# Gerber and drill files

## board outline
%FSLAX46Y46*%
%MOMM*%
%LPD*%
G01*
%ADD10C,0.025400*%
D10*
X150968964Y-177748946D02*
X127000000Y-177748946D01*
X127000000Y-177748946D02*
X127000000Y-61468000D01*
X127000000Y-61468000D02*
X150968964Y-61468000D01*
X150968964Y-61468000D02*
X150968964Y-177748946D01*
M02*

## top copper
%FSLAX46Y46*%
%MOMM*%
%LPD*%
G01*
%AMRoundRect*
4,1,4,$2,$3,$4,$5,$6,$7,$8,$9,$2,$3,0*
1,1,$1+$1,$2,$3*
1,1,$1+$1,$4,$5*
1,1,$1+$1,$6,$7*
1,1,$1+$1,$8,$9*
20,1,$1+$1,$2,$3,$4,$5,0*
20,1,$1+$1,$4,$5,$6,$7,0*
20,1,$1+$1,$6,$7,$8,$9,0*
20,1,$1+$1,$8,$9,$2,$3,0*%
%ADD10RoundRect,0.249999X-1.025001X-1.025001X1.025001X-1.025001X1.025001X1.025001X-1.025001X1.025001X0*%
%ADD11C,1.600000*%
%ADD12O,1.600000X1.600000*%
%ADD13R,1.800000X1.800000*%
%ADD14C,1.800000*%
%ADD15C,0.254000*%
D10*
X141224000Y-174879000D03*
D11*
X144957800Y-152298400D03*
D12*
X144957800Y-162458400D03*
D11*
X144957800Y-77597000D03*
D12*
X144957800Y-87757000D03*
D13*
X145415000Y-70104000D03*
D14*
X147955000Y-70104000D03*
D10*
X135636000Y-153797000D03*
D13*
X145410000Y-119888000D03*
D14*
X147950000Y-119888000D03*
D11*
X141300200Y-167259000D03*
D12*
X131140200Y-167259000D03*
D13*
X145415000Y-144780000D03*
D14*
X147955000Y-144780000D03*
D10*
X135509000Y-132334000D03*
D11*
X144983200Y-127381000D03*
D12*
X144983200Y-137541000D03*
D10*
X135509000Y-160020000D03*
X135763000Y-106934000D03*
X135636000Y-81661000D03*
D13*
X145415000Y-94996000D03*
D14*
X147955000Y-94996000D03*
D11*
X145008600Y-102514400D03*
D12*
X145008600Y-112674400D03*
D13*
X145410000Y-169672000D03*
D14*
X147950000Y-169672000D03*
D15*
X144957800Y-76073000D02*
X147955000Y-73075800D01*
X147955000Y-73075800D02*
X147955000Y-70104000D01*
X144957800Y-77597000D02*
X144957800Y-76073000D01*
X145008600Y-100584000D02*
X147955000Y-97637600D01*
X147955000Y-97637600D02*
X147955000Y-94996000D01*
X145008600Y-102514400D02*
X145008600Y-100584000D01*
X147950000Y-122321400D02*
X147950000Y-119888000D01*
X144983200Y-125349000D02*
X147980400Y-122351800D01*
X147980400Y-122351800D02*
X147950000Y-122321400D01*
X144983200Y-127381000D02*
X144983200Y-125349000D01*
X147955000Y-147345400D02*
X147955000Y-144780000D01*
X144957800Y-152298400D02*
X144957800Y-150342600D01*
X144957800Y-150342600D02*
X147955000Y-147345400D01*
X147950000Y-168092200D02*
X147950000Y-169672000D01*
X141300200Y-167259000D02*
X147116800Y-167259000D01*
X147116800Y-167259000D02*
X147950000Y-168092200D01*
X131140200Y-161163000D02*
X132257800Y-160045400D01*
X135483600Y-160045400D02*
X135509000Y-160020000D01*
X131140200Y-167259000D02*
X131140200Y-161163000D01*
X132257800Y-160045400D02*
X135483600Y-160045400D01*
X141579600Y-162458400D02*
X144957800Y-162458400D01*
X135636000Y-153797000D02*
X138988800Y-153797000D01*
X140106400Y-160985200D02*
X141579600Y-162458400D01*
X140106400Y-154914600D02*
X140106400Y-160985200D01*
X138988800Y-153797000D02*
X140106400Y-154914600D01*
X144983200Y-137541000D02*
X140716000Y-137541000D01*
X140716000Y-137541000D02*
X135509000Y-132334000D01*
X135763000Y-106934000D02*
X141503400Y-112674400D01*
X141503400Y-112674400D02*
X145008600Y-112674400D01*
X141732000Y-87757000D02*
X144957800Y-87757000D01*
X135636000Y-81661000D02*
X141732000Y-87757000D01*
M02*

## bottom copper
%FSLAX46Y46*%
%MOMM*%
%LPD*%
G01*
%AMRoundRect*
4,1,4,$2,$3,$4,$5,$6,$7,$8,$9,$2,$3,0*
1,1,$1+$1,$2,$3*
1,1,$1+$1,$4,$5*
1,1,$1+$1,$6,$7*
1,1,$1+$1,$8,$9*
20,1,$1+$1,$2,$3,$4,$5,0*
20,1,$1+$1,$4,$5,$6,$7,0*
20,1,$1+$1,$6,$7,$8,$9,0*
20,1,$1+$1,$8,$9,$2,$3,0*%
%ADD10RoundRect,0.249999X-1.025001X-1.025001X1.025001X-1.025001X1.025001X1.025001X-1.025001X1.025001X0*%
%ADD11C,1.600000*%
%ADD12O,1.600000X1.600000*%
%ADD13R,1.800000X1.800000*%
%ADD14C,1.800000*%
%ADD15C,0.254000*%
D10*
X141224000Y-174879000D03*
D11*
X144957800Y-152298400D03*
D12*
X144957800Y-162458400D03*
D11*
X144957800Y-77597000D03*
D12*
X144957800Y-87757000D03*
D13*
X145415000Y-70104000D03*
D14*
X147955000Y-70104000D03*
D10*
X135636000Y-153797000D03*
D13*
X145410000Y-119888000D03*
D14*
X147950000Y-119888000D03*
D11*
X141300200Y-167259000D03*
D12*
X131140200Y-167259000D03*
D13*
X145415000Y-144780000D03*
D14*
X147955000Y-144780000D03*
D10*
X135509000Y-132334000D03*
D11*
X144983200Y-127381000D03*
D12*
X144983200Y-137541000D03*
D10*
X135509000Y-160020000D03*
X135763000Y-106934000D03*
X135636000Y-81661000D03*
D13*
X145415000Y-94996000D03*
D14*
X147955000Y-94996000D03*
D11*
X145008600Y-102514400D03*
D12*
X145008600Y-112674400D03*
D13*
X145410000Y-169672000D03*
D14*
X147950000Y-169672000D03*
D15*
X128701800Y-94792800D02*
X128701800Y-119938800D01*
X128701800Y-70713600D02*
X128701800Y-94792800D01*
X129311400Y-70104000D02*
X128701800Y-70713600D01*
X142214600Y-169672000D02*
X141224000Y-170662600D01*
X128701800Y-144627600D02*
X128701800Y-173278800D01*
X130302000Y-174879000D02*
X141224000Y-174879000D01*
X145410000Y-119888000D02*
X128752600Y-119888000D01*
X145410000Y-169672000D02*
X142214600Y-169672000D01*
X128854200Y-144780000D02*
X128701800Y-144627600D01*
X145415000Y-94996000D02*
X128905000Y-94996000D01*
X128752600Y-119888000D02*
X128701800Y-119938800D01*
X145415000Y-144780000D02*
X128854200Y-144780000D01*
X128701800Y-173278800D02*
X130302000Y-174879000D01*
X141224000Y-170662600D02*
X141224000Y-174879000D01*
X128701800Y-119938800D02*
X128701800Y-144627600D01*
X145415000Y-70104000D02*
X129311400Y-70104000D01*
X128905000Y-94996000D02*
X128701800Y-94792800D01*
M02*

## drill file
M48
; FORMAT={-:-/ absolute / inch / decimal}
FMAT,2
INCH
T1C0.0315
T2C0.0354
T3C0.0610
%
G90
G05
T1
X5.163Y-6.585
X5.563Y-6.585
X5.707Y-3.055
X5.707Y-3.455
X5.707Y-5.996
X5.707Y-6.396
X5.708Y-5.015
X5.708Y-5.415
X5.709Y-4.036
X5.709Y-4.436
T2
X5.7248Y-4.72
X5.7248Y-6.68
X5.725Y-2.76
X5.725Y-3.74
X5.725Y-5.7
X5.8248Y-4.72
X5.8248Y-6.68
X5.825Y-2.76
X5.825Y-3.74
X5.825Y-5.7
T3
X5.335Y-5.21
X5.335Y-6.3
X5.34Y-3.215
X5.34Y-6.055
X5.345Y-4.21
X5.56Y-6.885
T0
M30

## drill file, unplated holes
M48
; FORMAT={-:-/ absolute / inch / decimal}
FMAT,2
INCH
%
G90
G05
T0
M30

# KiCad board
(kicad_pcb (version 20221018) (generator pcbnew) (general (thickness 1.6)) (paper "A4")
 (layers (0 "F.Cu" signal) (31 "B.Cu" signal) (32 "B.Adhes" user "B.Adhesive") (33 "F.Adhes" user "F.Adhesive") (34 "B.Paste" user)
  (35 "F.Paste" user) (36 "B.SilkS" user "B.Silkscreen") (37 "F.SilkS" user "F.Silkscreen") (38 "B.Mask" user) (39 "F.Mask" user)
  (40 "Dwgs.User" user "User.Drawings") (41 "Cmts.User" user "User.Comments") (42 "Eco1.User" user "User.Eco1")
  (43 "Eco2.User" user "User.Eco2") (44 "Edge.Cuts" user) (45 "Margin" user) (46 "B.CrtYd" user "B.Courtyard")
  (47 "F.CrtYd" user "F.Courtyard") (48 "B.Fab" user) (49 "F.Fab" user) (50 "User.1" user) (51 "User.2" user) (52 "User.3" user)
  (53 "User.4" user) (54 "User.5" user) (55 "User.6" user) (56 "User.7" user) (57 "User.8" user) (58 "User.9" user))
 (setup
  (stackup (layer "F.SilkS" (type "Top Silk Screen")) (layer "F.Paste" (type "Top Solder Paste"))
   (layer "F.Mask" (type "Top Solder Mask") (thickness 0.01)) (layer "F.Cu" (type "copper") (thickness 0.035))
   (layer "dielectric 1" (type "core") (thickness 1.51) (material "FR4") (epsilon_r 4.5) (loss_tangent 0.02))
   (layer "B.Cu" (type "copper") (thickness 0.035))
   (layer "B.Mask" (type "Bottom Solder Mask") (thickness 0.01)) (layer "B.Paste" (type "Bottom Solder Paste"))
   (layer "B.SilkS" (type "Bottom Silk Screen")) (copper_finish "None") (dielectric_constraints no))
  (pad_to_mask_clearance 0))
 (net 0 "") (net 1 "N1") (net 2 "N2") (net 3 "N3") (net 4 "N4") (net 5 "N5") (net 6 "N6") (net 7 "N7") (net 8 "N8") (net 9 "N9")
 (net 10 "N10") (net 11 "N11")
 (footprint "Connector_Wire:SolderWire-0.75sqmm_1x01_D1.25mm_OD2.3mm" (layer "F.Cu") (at 141.224 174.879)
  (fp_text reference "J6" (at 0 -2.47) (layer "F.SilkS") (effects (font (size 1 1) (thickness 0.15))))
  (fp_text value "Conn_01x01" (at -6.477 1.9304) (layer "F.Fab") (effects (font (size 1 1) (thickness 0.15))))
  (pad "1" thru_hole roundrect (at 0 0) (size 2.55 2.55) (drill 1.55) (layers "*.Cu" "*.Mask") (roundrect_rratio 0.09803882353) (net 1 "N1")))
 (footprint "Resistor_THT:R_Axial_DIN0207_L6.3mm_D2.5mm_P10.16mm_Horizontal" (layer "F.Cu") (at 144.9578 152.2984 -90)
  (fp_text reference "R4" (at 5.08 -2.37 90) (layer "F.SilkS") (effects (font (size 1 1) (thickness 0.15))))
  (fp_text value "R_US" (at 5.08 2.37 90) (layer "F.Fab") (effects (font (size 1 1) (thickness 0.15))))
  (pad "1" thru_hole circle (at 0 0 270) (size 1.6 1.6) (drill 0.8) (layers "*.Cu" "*.Mask") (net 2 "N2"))
  (pad "2" thru_hole oval (at 10.16 0 270) (size 1.6 1.6) (drill 0.8) (layers "*.Cu" "*.Mask") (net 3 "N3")))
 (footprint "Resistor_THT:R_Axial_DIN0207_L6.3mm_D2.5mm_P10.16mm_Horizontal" (layer "F.Cu") (at 144.9578 77.597 -90)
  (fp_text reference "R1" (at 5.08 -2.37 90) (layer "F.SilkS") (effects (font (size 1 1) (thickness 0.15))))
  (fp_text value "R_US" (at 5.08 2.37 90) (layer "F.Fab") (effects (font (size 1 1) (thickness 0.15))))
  (pad "1" thru_hole circle (at 0 0 270) (size 1.6 1.6) (drill 0.8) (layers "*.Cu" "*.Mask") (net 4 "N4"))
  (pad "2" thru_hole oval (at 10.16 0 270) (size 1.6 1.6) (drill 0.8) (layers "*.Cu" "*.Mask") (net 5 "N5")))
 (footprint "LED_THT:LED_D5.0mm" (layer "F.Cu") (at 145.415 70.104)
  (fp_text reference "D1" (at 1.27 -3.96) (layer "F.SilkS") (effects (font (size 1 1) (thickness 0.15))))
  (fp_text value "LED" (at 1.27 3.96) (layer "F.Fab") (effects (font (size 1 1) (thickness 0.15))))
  (pad "1" thru_hole rect (at 0 0) (size 1.8 1.8) (drill 0.9) (layers "*.Cu" "*.Mask") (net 1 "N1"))
  (pad "2" thru_hole circle (at 2.54 0) (size 1.8 1.8) (drill 0.9) (layers "*.Cu" "*.Mask") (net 4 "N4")))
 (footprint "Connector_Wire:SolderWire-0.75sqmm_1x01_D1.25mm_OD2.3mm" (layer "F.Cu") (at 135.636 153.797)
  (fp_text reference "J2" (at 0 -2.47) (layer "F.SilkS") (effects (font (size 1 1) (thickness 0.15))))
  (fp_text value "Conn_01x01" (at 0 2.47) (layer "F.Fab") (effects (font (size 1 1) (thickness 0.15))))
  (pad "1" thru_hole roundrect (at 0 0) (size 2.55 2.55) (drill 1.55) (layers "*.Cu" "*.Mask") (roundrect_rratio 0.09803882353) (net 3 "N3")))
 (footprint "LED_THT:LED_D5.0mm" (layer "F.Cu") (at 145.41 119.888)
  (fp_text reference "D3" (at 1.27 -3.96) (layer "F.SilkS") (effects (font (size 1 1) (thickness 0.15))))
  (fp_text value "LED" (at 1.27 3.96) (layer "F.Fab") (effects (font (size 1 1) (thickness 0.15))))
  (pad "1" thru_hole rect (at 0 0) (size 1.8 1.8) (drill 0.9) (layers "*.Cu" "*.Mask") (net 1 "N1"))
  (pad "2" thru_hole circle (at 2.54 0) (size 1.8 1.8) (drill 0.9) (layers "*.Cu" "*.Mask") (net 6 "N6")))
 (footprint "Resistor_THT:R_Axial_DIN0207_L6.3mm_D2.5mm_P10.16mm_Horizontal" (layer "F.Cu") (at 141.3002 167.259 180)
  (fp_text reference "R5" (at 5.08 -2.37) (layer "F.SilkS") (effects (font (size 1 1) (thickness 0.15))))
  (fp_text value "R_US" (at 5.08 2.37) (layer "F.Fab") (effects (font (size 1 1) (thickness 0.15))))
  (pad "1" thru_hole circle (at 0 0 180) (size 1.6 1.6) (drill 0.8) (layers "*.Cu" "*.Mask") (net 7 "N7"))
  (pad "2" thru_hole oval (at 10.16 0 180) (size 1.6 1.6) (drill 0.8) (layers "*.Cu" "*.Mask") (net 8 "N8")))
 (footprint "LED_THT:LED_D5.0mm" (layer "F.Cu") (at 145.415 144.78)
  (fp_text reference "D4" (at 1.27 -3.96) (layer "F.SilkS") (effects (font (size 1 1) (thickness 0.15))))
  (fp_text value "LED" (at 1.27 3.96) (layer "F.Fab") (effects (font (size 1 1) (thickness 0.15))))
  (pad "1" thru_hole rect (at 0 0) (size 1.8 1.8) (drill 0.9) (layers "*.Cu" "*.Mask") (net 1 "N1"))
  (pad "2" thru_hole circle (at 2.54 0) (size 1.8 1.8) (drill 0.9) (layers "*.Cu" "*.Mask") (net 2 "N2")))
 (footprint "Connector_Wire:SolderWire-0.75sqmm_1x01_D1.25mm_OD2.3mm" (layer "F.Cu") (at 135.509 132.334)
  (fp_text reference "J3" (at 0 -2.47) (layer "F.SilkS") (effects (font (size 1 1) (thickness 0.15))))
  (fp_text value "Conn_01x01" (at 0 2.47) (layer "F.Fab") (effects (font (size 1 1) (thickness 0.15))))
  (pad "1" thru_hole roundrect (at 0 0) (size 2.55 2.55) (drill 1.55) (layers "*.Cu" "*.Mask") (roundrect_rratio 0.09803882353) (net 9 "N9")))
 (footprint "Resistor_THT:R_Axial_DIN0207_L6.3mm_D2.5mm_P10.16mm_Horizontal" (layer "F.Cu") (at 144.9832 127.381 -90)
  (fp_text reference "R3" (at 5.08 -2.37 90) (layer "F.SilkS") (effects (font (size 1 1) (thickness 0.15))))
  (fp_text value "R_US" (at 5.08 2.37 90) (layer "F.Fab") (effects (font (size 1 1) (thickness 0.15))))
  (pad "1" thru_hole circle (at 0 0 270) (size 1.6 1.6) (drill 0.8) (layers "*.Cu" "*.Mask") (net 6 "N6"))
  (pad "2" thru_hole oval (at 10.16 0 270) (size 1.6 1.6) (drill 0.8) (layers "*.Cu" "*.Mask") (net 9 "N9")))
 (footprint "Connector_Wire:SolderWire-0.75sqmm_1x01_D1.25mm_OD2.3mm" (layer "F.Cu") (at 135.509 160.02)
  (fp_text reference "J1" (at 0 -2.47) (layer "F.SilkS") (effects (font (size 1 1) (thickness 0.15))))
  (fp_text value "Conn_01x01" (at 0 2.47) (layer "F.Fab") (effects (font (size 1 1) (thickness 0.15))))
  (pad "1" thru_hole roundrect (at 0 0) (size 2.55 2.55) (drill 1.55) (layers "*.Cu" "*.Mask") (roundrect_rratio 0.09803882353) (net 8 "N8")))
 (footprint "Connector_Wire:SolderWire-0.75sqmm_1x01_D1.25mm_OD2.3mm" (layer "F.Cu") (at 135.763 106.934)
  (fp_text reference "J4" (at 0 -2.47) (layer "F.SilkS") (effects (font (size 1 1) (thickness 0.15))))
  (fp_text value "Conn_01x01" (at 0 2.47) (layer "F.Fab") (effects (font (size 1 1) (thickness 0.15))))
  (pad "1" thru_hole roundrect (at 0 0) (size 2.55 2.55) (drill 1.55) (layers "*.Cu" "*.Mask") (roundrect_rratio 0.09803882353)
   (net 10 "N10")))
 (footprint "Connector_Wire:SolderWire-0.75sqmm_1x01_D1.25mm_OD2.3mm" (layer "F.Cu") (at 135.636 81.661)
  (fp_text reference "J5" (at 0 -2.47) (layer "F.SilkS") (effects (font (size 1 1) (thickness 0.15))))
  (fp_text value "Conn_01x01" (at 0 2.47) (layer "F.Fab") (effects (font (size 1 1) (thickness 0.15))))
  (pad "1" thru_hole roundrect (at 0 0) (size 2.55 2.55) (drill 1.55) (layers "*.Cu" "*.Mask") (roundrect_rratio 0.09803882353) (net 5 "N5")))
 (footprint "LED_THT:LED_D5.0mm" (layer "F.Cu") (at 145.415 94.996)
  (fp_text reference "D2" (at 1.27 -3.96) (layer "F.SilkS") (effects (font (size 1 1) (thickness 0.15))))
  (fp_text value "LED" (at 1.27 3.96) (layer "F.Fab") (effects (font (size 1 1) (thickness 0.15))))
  (pad "1" thru_hole rect (at 0 0) (size 1.8 1.8) (drill 0.9) (layers "*.Cu" "*.Mask") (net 1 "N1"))
  (pad "2" thru_hole circle (at 2.54 0) (size 1.8 1.8) (drill 0.9) (layers "*.Cu" "*.Mask") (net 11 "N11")))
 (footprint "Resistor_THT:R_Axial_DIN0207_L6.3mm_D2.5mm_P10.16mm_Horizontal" (layer "F.Cu") (at 145.0086 102.5144 -90)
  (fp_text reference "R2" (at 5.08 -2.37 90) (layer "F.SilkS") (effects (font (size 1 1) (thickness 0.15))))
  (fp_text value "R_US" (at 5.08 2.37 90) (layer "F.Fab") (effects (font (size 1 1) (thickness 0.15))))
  (pad "1" thru_hole circle (at 0 0 270) (size 1.6 1.6) (drill 0.8) (layers "*.Cu" "*.Mask") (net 11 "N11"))
  (pad "2" thru_hole oval (at 10.16 0 270) (size 1.6 1.6) (drill 0.8) (layers "*.Cu" "*.Mask") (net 10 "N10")))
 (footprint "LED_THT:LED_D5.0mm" (layer "F.Cu") (at 145.41 169.672)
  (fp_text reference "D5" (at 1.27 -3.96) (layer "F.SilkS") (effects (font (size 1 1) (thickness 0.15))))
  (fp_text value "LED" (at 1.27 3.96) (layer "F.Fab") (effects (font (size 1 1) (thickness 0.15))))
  (pad "1" thru_hole rect (at 0 0) (size 1.8 1.8) (drill 0.9) (layers "*.Cu" "*.Mask") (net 1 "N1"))
  (pad "2" thru_hole circle (at 2.54 0) (size 1.8 1.8) (drill 0.9) (layers "*.Cu" "*.Mask") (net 7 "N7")))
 (gr_line (start 150.968964 177.748946) (end 127 177.748946) (stroke (width 0.0254) (type default)) (layer "Edge.Cuts"))
 (gr_line (start 127 177.748946) (end 127 61.468) (stroke (width 0.0254) (type default)) (layer "Edge.Cuts"))
 (gr_line (start 127 61.468) (end 150.968964 61.468) (stroke (width 0.0254) (type default)) (layer "Edge.Cuts"))
 (gr_line (start 150.968964 61.468) (end 150.968964 177.748946) (stroke (width 0.0254) (type default)) (layer "Edge.Cuts"))
 (segment (start 128.7018 94.7928) (end 128.7018 119.9388) (width 0.254) (layer "B.Cu") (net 1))
 (segment (start 128.7018 70.7136) (end 128.7018 94.7928) (width 0.254) (layer "B.Cu") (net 1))
 (segment (start 129.3114 70.104) (end 128.7018 70.7136) (width 0.254) (layer "B.Cu") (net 1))
 (segment (start 142.2146 169.672) (end 141.224 170.6626) (width 0.254) (layer "B.Cu") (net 1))
 (segment (start 128.7018 144.6276) (end 128.7018 173.2788) (width 0.254) (layer "B.Cu") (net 1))
 (segment (start 130.302 174.879) (end 141.224 174.879) (width 0.254) (layer "B.Cu") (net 1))
 (segment (start 145.41 119.888) (end 128.7526 119.888) (width 0.254) (layer "B.Cu") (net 1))
 (segment (start 145.41 169.672) (end 142.2146 169.672) (width 0.254) (layer "B.Cu") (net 1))
 (segment (start 128.8542 144.78) (end 128.7018 144.6276) (width 0.254) (layer "B.Cu") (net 1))
 (segment (start 145.415 94.996) (end 128.905 94.996) (width 0.254) (layer "B.Cu") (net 1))
 (segment (start 128.7526 119.888) (end 128.7018 119.9388) (width 0.254) (layer "B.Cu") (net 1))
 (segment (start 145.415 144.78) (end 128.8542 144.78) (width 0.254) (layer "B.Cu") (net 1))
 (segment (start 128.7018 173.2788) (end 130.302 174.879) (width 0.254) (layer "B.Cu") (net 1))
 (segment (start 141.224 170.6626) (end 141.224 174.879) (width 0.254) (layer "B.Cu") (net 1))
 (segment (start 128.7018 119.9388) (end 128.7018 144.6276) (width 0.254) (layer "B.Cu") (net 1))
 (segment (start 145.415 70.104) (end 129.3114 70.104) (width 0.254) (layer "B.Cu") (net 1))
 (segment (start 128.905 94.996) (end 128.7018 94.7928) (width 0.254) (layer "B.Cu") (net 1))
 (segment (start 144.9578 76.073) (end 147.955 73.0758) (width 0.254) (layer "F.Cu") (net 4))
 (segment (start 147.955 73.0758) (end 147.955 70.104) (width 0.254) (layer "F.Cu") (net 4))
 (segment (start 144.9578 77.597) (end 144.9578 76.073) (width 0.254) (layer "F.Cu") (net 4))
 (segment (start 145.0086 100.584) (end 147.955 97.6376) (width 0.254) (layer "F.Cu") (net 11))
 (segment (start 147.955 97.6376) (end 147.955 94.996) (width 0.254) (layer "F.Cu") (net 11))
 (segment (start 145.0086 102.5144) (end 145.0086 100.584) (width 0.254) (layer "F.Cu") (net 11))
 (segment (start 147.95 122.3214) (end 147.95 119.888) (width 0.254) (layer "F.Cu") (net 6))
 (segment (start 144.9832 125.349) (end 147.9804 122.3518) (width 0.254) (layer "F.Cu") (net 6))
 (segment (start 147.9804 122.3518) (end 147.95 122.3214) (width 0.254) (layer "F.Cu") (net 6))
 (segment (start 144.9832 127.381) (end 144.9832 125.349) (width 0.254) (layer "F.Cu") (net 6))
 (segment (start 147.955 147.3454) (end 147.955 144.78) (width 0.254) (layer "F.Cu") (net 2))
 (segment (start 144.9578 152.2984) (end 144.9578 150.3426) (width 0.254) (layer "F.Cu") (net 2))
 (segment (start 144.9578 150.3426) (end 147.955 147.3454) (width 0.254) (layer "F.Cu") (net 2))
 (segment (start 147.95 168.0922) (end 147.95 169.672) (width 0.254) (layer "F.Cu") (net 7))
 (segment (start 141.3002 167.259) (end 147.1168 167.259) (width 0.254) (layer "F.Cu") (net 7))
 (segment (start 147.1168 167.259) (end 147.95 168.0922) (width 0.254) (layer "F.Cu") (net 7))
 (segment (start 131.1402 161.163) (end 132.2578 160.0454) (width 0.254) (layer "F.Cu") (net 8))
 (segment (start 135.4836 160.0454) (end 135.509 160.02) (width 0.254) (layer "F.Cu") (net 8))
 (segment (start 131.1402 167.259) (end 131.1402 161.163) (width 0.254) (layer "F.Cu") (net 8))
 (segment (start 132.2578 160.0454) (end 135.4836 160.0454) (width 0.254) (layer "F.Cu") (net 8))
 (segment (start 141.5796 162.4584) (end 144.9578 162.4584) (width 0.254) (layer "F.Cu") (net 3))
 (segment (start 135.636 153.797) (end 138.9888 153.797) (width 0.254) (layer "F.Cu") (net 3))
 (segment (start 140.1064 160.9852) (end 141.5796 162.4584) (width 0.254) (layer "F.Cu") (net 3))
 (segment (start 140.1064 154.9146) (end 140.1064 160.9852) (width 0.254) (layer "F.Cu") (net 3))
 (segment (start 138.9888 153.797) (end 140.1064 154.9146) (width 0.254) (layer "F.Cu") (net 3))
 (segment (start 144.9832 137.541) (end 140.716 137.541) (width 0.254) (layer "F.Cu") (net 9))
 (segment (start 140.716 137.541) (end 135.509 132.334) (width 0.254) (layer "F.Cu") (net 9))
 (segment (start 135.763 106.934) (end 141.5034 112.6744) (width 0.254) (layer "F.Cu") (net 10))
 (segment (start 141.5034 112.6744) (end 145.0086 112.6744) (width 0.254) (layer "F.Cu") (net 10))
 (segment (start 141.732 87.757) (end 144.9578 87.757) (width 0.254) (layer "F.Cu") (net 5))
 (segment (start 135.636 81.661) (end 141.732 87.757) (width 0.254) (layer "F.Cu") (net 5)))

